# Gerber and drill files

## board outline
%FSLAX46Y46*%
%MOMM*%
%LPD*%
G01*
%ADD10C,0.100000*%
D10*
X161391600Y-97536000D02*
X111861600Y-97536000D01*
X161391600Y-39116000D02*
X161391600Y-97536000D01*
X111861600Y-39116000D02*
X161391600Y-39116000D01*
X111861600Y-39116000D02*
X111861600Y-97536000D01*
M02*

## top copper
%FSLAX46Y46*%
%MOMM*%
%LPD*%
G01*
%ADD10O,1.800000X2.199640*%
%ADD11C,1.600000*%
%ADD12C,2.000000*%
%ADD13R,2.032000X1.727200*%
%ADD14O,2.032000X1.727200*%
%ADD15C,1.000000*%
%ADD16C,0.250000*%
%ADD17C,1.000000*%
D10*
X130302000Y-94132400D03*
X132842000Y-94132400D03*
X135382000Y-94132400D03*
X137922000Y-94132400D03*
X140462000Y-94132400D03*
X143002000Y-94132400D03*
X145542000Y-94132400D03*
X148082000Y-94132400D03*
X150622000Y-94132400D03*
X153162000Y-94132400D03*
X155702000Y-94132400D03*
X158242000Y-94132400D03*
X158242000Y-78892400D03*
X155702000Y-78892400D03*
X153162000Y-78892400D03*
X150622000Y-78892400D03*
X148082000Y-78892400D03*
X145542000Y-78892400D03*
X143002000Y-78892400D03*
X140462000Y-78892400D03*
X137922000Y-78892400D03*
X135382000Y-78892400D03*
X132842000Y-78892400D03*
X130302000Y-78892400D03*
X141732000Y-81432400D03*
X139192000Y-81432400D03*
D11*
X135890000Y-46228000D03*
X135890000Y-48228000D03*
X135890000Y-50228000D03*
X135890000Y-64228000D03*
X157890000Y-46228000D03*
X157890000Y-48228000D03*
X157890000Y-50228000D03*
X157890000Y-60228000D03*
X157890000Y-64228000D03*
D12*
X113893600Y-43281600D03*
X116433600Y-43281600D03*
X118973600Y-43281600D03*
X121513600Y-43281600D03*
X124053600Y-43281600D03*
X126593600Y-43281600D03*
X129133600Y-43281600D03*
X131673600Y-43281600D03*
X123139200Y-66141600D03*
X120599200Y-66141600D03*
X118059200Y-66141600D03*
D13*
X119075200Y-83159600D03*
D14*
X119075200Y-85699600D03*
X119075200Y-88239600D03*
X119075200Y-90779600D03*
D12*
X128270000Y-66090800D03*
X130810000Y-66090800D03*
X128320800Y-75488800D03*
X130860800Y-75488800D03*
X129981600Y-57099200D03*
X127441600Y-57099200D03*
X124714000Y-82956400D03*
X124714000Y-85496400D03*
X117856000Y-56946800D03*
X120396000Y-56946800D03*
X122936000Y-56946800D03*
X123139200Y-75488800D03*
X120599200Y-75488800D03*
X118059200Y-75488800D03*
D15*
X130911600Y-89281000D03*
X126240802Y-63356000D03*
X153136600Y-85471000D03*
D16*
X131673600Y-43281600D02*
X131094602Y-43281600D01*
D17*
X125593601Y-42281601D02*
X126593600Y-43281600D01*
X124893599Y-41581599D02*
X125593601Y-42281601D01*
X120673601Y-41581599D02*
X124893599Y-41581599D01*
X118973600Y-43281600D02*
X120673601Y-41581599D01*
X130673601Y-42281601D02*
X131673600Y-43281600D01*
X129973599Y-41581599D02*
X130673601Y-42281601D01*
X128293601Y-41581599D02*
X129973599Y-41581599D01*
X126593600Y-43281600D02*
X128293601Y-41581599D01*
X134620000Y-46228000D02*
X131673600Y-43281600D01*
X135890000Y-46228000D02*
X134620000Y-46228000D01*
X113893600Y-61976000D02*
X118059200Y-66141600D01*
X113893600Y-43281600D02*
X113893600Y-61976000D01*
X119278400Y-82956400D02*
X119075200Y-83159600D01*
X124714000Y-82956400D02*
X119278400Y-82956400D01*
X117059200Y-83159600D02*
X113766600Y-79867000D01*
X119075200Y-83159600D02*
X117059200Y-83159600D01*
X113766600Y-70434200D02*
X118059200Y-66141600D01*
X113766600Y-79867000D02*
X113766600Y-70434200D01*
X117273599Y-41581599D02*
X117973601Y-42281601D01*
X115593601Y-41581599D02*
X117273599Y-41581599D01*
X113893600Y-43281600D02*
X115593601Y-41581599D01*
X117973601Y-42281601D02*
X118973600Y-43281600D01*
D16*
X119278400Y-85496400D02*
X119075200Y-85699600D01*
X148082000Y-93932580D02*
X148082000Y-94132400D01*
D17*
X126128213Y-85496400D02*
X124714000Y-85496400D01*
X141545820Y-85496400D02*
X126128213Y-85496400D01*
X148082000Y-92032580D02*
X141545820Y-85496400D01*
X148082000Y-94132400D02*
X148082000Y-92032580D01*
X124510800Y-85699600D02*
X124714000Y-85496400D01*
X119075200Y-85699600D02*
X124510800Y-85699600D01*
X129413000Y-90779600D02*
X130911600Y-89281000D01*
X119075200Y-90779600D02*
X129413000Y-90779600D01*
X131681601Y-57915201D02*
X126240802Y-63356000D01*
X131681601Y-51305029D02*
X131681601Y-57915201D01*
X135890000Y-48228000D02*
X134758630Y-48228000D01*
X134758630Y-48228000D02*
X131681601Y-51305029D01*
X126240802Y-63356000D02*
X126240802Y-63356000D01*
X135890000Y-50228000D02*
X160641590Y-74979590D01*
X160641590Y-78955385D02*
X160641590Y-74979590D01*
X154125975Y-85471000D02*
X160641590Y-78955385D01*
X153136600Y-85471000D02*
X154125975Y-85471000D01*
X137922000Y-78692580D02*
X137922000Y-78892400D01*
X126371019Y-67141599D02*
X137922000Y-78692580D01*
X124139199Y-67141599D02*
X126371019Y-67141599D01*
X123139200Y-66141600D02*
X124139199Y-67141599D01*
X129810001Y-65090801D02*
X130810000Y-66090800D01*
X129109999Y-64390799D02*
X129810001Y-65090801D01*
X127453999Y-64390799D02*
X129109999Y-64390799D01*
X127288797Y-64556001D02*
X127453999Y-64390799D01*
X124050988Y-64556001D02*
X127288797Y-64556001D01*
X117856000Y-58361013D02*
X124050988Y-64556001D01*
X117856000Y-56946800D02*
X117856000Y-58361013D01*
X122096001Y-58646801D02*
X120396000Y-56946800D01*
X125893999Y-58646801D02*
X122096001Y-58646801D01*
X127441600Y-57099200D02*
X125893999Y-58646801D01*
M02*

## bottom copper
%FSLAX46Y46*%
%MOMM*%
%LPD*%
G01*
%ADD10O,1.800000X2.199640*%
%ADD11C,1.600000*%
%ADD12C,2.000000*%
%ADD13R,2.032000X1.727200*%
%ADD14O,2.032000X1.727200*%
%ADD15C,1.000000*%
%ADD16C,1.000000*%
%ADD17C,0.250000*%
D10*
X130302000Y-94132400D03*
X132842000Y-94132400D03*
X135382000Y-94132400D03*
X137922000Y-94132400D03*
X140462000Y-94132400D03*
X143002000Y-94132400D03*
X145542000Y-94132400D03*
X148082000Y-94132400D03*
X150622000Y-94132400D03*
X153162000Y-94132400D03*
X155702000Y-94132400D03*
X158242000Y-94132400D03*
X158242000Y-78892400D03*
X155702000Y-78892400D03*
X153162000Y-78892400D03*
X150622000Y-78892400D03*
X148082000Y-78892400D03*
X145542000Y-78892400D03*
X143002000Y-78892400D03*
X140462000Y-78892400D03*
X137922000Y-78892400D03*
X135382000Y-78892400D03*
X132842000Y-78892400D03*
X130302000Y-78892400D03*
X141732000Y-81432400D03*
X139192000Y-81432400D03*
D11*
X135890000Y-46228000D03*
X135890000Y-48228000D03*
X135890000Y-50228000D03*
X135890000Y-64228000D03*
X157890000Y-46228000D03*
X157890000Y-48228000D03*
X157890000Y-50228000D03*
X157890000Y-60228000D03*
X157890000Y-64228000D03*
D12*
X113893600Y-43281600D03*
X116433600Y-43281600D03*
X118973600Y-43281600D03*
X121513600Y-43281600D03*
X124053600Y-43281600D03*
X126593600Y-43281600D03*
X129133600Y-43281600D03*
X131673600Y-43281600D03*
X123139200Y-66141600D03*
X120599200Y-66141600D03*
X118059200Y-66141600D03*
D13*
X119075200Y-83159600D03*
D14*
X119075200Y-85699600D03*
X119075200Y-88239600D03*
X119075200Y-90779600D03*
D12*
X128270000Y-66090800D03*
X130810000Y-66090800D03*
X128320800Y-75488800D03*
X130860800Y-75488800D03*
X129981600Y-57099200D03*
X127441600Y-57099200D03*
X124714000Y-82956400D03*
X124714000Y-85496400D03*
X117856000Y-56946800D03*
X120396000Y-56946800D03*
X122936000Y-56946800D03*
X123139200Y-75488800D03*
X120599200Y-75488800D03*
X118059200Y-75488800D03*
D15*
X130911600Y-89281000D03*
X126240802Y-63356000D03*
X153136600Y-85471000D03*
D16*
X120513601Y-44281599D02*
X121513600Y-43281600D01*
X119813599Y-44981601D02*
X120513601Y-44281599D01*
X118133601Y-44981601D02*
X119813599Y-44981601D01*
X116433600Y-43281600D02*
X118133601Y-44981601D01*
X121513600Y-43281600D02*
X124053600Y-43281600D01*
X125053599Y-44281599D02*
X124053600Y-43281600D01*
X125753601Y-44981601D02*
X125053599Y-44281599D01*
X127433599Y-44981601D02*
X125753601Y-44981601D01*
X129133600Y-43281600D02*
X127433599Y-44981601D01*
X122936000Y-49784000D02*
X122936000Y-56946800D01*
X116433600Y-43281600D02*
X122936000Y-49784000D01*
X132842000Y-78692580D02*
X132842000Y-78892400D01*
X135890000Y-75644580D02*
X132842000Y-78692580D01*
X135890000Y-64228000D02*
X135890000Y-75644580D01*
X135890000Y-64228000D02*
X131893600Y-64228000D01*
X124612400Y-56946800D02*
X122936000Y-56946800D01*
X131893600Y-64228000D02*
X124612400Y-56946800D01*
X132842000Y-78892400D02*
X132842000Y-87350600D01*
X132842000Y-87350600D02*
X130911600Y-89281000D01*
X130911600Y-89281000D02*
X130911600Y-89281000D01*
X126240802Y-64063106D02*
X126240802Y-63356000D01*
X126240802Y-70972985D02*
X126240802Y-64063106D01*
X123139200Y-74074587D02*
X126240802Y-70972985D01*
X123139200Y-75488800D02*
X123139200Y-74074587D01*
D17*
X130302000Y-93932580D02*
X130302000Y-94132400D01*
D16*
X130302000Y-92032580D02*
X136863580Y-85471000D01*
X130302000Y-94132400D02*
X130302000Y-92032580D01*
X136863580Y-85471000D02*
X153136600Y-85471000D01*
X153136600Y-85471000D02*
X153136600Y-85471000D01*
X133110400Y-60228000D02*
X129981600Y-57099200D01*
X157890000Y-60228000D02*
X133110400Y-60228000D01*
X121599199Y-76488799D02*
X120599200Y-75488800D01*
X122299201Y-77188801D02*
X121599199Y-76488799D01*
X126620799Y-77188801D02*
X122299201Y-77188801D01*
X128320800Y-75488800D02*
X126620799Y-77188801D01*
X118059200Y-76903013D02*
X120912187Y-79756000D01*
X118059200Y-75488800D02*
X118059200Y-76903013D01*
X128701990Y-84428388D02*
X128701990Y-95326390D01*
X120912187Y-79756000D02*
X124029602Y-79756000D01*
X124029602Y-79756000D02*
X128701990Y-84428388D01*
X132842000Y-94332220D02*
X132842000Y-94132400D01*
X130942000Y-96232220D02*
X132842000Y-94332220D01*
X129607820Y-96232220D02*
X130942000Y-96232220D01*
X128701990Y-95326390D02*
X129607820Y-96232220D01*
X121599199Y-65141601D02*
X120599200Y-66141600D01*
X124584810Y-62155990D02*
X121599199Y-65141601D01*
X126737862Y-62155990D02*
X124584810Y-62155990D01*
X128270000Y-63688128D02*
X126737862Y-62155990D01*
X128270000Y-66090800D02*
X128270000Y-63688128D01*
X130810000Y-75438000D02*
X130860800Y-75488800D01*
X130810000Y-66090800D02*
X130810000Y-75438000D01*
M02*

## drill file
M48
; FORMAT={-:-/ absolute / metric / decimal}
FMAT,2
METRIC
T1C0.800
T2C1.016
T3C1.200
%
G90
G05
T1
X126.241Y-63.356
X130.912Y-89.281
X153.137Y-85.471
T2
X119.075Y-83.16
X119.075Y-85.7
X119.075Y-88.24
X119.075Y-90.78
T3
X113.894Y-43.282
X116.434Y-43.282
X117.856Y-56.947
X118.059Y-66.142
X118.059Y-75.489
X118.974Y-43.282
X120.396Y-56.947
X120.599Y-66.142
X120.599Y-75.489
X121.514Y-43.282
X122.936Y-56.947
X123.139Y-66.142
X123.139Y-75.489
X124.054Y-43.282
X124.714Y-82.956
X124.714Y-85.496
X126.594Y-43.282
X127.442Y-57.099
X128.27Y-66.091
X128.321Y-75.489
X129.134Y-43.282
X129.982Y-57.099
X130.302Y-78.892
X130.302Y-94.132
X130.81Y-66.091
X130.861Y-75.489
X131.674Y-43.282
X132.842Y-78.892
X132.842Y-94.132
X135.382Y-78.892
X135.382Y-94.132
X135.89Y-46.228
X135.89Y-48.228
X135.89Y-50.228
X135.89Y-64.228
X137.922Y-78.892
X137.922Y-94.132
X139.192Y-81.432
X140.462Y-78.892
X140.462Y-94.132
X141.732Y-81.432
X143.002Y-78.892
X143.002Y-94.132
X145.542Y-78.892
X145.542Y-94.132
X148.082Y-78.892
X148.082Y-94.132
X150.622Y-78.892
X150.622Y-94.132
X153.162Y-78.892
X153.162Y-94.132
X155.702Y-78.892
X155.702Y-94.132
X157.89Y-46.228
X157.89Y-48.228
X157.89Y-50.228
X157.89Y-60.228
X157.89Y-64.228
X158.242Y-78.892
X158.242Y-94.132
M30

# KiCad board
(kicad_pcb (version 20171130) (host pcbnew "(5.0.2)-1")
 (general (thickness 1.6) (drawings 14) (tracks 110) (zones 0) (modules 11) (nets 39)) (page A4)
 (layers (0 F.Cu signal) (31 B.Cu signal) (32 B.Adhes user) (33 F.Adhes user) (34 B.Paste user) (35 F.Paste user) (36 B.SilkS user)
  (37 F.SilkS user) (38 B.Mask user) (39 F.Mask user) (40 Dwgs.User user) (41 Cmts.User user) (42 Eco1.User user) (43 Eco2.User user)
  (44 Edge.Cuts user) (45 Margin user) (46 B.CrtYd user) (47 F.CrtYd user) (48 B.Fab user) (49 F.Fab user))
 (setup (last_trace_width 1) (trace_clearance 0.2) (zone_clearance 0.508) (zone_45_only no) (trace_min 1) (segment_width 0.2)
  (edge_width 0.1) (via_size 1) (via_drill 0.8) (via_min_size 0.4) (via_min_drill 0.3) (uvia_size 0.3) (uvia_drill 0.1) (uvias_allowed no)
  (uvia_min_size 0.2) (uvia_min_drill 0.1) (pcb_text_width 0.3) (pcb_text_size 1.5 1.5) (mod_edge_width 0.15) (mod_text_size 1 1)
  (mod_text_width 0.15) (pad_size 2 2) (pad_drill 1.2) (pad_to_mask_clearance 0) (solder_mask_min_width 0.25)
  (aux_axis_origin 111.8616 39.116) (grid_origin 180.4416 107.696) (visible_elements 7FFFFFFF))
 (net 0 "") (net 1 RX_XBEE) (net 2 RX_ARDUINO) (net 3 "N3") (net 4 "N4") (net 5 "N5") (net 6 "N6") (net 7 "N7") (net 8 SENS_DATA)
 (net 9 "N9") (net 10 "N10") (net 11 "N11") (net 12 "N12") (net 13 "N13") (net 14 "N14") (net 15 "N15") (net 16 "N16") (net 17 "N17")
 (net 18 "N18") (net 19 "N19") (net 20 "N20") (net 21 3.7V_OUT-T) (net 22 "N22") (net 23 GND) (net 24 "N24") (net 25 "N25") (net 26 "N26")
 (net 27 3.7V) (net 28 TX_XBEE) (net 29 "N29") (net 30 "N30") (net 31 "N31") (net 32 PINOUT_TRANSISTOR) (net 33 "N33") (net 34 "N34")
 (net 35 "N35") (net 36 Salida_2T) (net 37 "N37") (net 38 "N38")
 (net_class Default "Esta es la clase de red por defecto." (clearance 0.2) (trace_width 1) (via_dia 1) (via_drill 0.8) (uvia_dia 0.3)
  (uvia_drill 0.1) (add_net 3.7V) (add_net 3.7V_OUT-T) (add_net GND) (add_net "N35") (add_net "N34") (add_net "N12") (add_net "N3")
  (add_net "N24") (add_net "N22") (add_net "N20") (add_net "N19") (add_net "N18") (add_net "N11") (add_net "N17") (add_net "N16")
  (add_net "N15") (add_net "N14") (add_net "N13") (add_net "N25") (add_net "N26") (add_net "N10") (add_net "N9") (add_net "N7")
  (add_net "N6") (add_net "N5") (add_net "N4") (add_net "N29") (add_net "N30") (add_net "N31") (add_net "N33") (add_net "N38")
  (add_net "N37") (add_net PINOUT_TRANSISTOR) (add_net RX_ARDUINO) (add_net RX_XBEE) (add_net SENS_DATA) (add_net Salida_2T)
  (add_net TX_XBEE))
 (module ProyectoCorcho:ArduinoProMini (layer F.Cu) (at 144.272 86.5124)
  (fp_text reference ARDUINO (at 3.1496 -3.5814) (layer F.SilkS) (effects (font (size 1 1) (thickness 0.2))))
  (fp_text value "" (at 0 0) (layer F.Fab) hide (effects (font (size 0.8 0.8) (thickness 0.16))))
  (pad 12 thru_hole oval (at -13.97 7.62) (size 1.8 2.19964) (drill 1.2) (layers *.Cu *.Mask) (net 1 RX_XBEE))
  (pad 11 thru_hole oval (at -11.43 7.62) (size 1.8 2.19964) (drill 1.2) (layers *.Cu *.Mask) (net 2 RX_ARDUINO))
  (pad 10 thru_hole oval (at -8.89 7.62) (size 1.8 2.19964) (drill 1.2) (layers *.Cu *.Mask) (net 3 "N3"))
  (pad 9 thru_hole oval (at -6.35 7.62) (size 1.8 2.19964) (drill 1.2) (layers *.Cu *.Mask) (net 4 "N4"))
  (pad 8 thru_hole oval (at -3.81 7.62) (size 1.8 2.19964) (drill 1.2) (layers *.Cu *.Mask) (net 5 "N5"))
  (pad 7 thru_hole oval (at -1.27 7.62) (size 1.8 2.19964) (drill 1.2) (layers *.Cu *.Mask) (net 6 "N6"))
  (pad 6 thru_hole oval (at 1.27 7.62) (size 1.8 2.19964) (drill 1.2) (layers *.Cu *.Mask) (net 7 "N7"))
  (pad 5 thru_hole oval (at 3.81 7.62) (size 1.8 2.19964) (drill 1.2) (layers *.Cu *.Mask) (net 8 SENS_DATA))
  (pad 4 thru_hole oval (at 6.35 7.62) (size 1.8 2.19964) (drill 1.2) (layers *.Cu *.Mask) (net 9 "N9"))
  (pad 3 thru_hole oval (at 8.89 7.62) (size 1.8 2.19964) (drill 1.2) (layers *.Cu *.Mask) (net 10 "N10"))
  (pad 2 thru_hole oval (at 11.43 7.62) (size 1.8 2.19964) (drill 1.2) (layers *.Cu *.Mask) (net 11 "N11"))
  (pad 1 thru_hole oval (at 13.97 7.62) (size 1.8 2.19964) (drill 1.2) (layers *.Cu *.Mask) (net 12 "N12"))
  (pad 24 thru_hole oval (at 13.97 -7.62) (size 1.8 2.19964) (drill 1.2) (layers *.Cu *.Mask) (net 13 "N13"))
  (pad 23 thru_hole oval (at 11.43 -7.62) (size 1.8 2.19964) (drill 1.2) (layers *.Cu *.Mask) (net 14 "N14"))
  (pad 22 thru_hole oval (at 8.89 -7.62) (size 1.8 2.19964) (drill 1.2) (layers *.Cu *.Mask) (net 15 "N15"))
  (pad 21 thru_hole oval (at 6.35 -7.62) (size 1.8 2.19964) (drill 1.2) (layers *.Cu *.Mask) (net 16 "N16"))
  (pad 20 thru_hole oval (at 3.81 -7.62) (size 1.8 2.19964) (drill 1.2) (layers *.Cu *.Mask) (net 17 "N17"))
  (pad 19 thru_hole oval (at 1.27 -7.62) (size 1.8 2.19964) (drill 1.2) (layers *.Cu *.Mask) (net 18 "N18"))
  (pad 18 thru_hole oval (at -1.27 -7.62) (size 1.8 2.19964) (drill 1.2) (layers *.Cu *.Mask) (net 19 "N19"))
  (pad 17 thru_hole oval (at -3.81 -7.62) (size 1.8 2.19964) (drill 1.2) (layers *.Cu *.Mask) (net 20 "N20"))
  (pad 16 thru_hole oval (at -6.35 -7.62) (size 1.8 2.19964) (drill 1.2) (layers *.Cu *.Mask) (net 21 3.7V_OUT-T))
  (pad 15 thru_hole oval (at -8.89 -7.62) (size 1.8 2.19964) (drill 1.2) (layers *.Cu *.Mask) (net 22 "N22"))
  (pad 14 thru_hole oval (at -11.43 -7.62) (size 1.8 2.19964) (drill 1.2) (layers *.Cu *.Mask) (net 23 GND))
  (pad 13 thru_hole oval (at -13.97 -7.62) (size 1.8 2.19964) (drill 1.2) (layers *.Cu *.Mask) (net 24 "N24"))
  (pad 25 thru_hole oval (at -2.54 -5.08) (size 1.8 2.19964) (drill 1.2) (layers *.Cu *.Mask) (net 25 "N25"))
  (pad 26 thru_hole oval (at -5.08 -5.08) (size 1.8 2.19964) (drill 1.2) (layers *.Cu *.Mask) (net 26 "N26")))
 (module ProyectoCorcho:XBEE (layer F.Cu) (at 134.62 44.958)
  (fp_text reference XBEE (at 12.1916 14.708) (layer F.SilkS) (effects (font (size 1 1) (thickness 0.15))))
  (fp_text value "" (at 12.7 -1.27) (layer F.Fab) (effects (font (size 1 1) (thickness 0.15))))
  (pad 1 thru_hole circle (at 1.27 1.27) (size 1.6 1.6) (drill 1.2) (layers *.Cu *.Mask) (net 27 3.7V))
  (pad 2 thru_hole circle (at 1.27 3.27) (size 1.6 1.6) (drill 1.2) (layers *.Cu *.Mask) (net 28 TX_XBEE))
  (pad 3 thru_hole circle (at 1.27 5.27) (size 1.6 1.6) (drill 1.2) (layers *.Cu *.Mask) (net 1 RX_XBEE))
  (pad 4 thru_hole circle (at 1.27 19.27) (size 1.6 1.6) (drill 1.2) (layers *.Cu *.Mask) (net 23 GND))
  (pad 5 thru_hole circle (at 23.27 1.27) (size 1.6 1.6) (drill 1.2) (layers *.Cu *.Mask) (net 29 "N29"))
  (pad 6 thru_hole circle (at 23.27 3.27) (size 1.6 1.6) (drill 1.2) (layers *.Cu *.Mask) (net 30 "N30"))
  (pad 7 thru_hole circle (at 23.27 5.27) (size 1.6 1.6) (drill 1.2) (layers *.Cu *.Mask) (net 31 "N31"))
  (pad 8 thru_hole circle (at 23.27 15.27) (size 1.6 1.6) (drill 1.2) (layers *.Cu *.Mask) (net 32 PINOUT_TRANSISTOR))
  (pad 9 thru_hole circle (at 23.27 19.27) (size 1.6 1.6) (drill 1.2) (layers *.Cu *.Mask) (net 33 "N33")))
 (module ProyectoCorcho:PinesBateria (layer F.Cu) (at 112.6236 42.0116)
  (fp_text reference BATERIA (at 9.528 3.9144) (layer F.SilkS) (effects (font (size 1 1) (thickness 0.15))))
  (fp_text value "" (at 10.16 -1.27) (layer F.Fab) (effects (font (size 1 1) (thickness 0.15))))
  (pad 1 thru_hole circle (at 1.27 1.27) (size 2 2) (drill 1.2) (layers *.Cu *.Mask) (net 27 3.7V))
  (pad 2 thru_hole circle (at 3.81 1.27) (size 2 2) (drill 1.2) (layers *.Cu *.Mask) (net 23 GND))
  (pad 3 thru_hole circle (at 6.35 1.27) (size 2 2) (drill 1.2) (layers *.Cu *.Mask) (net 27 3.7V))
  (pad 4 thru_hole circle (at 8.89 1.27) (size 2 2) (drill 1.2) (layers *.Cu *.Mask) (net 23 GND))
  (pad 5 thru_hole circle (at 11.43 1.27) (size 2 2) (drill 1.2) (layers *.Cu *.Mask) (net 23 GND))
  (pad 6 thru_hole circle (at 13.97 1.27) (size 2 2) (drill 1.2) (layers *.Cu *.Mask) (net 27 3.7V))
  (pad 7 thru_hole circle (at 16.51 1.27) (size 2 2) (drill 1.2) (layers *.Cu *.Mask) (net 23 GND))
  (pad 8 thru_hole circle (at 19.05 1.27) (size 2 2) (drill 1.2) (layers *.Cu *.Mask) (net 27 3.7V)))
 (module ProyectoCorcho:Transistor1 (layer B.Cu) (at 120.5992 66.1416)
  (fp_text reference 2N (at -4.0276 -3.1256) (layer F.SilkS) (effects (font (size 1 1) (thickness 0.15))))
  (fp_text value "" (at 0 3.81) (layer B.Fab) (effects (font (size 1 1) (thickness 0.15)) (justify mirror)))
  (pad 3 thru_hole circle (at 2.54 0) (size 2 2) (drill 1.2) (layers *.Cu *.Mask) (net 21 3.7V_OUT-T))
  (pad 2 thru_hole circle (at 0 0) (size 2 2) (drill 1.2) (layers *.Cu *.Mask) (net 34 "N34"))
  (pad 1 thru_hole circle (at -2.54 0) (size 2 2) (drill 1.2) (layers *.Cu *.Mask) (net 27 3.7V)))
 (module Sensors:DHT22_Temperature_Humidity (layer F.Cu) (at 119.0752 86.9696 270)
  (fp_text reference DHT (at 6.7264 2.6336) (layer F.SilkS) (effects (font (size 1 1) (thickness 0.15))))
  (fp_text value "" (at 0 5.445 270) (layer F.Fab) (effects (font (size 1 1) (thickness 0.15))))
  (pad 1 thru_hole rect (at -3.81 0) (size 2.032 1.7272) (drill 1.016) (layers *.Cu *.Mask F.SilkS) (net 27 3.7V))
  (pad 2 thru_hole oval (at -1.27 0) (size 2.032 1.7272) (drill 1.016) (layers *.Cu *.Mask F.SilkS) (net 8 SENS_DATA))
  (pad 3 thru_hole oval (at 1.27 0) (size 2.032 1.7272) (drill 1.016) (layers *.Cu *.Mask F.SilkS) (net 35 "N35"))
  (pad 4 thru_hole oval (at 3.81 0) (size 2.032 1.7272) (drill 1.016) (layers *.Cu *.Mask F.SilkS) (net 23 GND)))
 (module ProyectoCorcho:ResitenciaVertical (layer F.Cu) (at 128.27 66.0908)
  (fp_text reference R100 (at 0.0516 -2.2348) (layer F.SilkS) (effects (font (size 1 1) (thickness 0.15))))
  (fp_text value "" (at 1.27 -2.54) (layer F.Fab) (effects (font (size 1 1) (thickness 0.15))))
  (pad 1 thru_hole circle (at 0 0) (size 2 2) (drill 1.2) (layers *.Cu *.Mask) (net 34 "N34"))
  (pad 2 thru_hole circle (at 2.54 0) (size 2 2) (drill 1.2) (layers *.Cu *.Mask) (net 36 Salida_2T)))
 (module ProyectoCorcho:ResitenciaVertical (layer F.Cu) (at 128.3208 75.4888)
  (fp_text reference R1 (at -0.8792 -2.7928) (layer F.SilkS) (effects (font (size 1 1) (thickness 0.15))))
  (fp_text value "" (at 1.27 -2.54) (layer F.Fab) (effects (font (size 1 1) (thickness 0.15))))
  (pad 1 thru_hole circle (at 0 0) (size 2 2) (drill 1.2) (layers *.Cu *.Mask) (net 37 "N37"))
  (pad 2 thru_hole circle (at 2.54 0) (size 2 2) (drill 1.2) (layers *.Cu *.Mask) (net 36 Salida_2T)))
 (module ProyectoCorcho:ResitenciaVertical (layer F.Cu) (at 127.4416 57.0992)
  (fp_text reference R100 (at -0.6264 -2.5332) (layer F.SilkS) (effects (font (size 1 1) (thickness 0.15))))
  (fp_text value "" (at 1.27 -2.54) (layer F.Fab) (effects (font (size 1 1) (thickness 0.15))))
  (pad 2 thru_hole circle (at 2.54 0) (size 2 2) (drill 1.2) (layers *.Cu *.Mask) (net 32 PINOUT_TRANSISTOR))
  (pad 1 thru_hole circle (at 0 0) (size 2 2) (drill 1.2) (layers *.Cu *.Mask) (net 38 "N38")))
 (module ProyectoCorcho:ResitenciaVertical (layer F.Cu) (at 124.714 82.9564 270)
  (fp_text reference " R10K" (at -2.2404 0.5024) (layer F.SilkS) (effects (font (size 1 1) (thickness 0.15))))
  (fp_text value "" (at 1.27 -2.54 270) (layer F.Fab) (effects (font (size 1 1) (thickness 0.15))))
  (pad 1 thru_hole circle (at 0 0 270) (size 2 2) (drill 1.2) (layers *.Cu *.Mask) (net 27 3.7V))
  (pad 2 thru_hole circle (at 2.54 0 270) (size 2 2) (drill 1.2) (layers *.Cu *.Mask) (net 8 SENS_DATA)))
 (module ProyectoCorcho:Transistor (layer F.Cu) (at 120.396 56.9468)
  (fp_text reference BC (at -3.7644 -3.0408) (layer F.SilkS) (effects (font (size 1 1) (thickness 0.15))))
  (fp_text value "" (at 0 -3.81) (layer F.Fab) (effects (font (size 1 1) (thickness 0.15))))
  (pad 1 thru_hole circle (at -2.54 0) (size 2 2) (drill 1.2) (layers *.Cu *.Mask) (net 36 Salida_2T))
  (pad 2 thru_hole circle (at 0 0) (size 2 2) (drill 1.2) (layers *.Cu *.Mask) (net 38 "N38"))
  (pad 3 thru_hole circle (at 2.54 0) (size 2 2) (drill 1.2) (layers *.Cu *.Mask) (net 23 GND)))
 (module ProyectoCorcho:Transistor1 (layer B.Cu) (at 120.5992 75.4888 180)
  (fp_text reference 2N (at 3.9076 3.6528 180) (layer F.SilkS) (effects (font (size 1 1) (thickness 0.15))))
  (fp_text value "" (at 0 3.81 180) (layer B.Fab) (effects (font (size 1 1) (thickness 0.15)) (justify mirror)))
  (pad 1 thru_hole circle (at -2.54 0 180) (size 2 2) (drill 1.2) (layers *.Cu *.Mask) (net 28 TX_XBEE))
  (pad 2 thru_hole circle (at 0 0 180) (size 2 2) (drill 1.2) (layers *.Cu *.Mask) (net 37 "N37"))
  (pad 3 thru_hole circle (at 2.54 0 180) (size 2 2) (drill 1.2) (layers *.Cu *.Mask) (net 2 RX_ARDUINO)))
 (gr_line (start 161.3916 97.536) (end 111.8616 97.536) (layer Edge.Cuts) (width 0.1))
 (gr_line (start 161.3916 39.116) (end 161.3916 97.536) (layer Edge.Cuts) (width 0.1))
 (gr_line (start 111.8616 39.116) (end 161.3916 39.116) (layer Edge.Cuts) (width 0.1))
 (gr_line (start 111.8616 39.116) (end 111.8616 97.536) (layer Edge.Cuts) (width 0.1))
 (segment (start 131.6736 43.2816) (end 131.094602 43.2816) (width 0.25) (layer F.Cu) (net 27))
 (segment (start 125.593601 42.281601) (end 126.5936 43.2816) (width 1) (layer F.Cu) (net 27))
 (segment (start 124.893599 41.581599) (end 125.593601 42.281601) (width 1) (layer F.Cu) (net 27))
 (segment (start 120.673601 41.581599) (end 124.893599 41.581599) (width 1) (layer F.Cu) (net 27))
 (segment (start 118.9736 43.2816) (end 120.673601 41.581599) (width 1) (layer F.Cu) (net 27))
 (segment (start 130.673601 42.281601) (end 131.6736 43.2816) (width 1) (layer F.Cu) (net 27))
 (segment (start 129.973599 41.581599) (end 130.673601 42.281601) (width 1) (layer F.Cu) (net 27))
 (segment (start 128.293601 41.581599) (end 129.973599 41.581599) (width 1) (layer F.Cu) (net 27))
 (segment (start 126.5936 43.2816) (end 128.293601 41.581599) (width 1) (layer F.Cu) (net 27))
 (segment (start 134.62 46.228) (end 131.6736 43.2816) (width 1) (layer F.Cu) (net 27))
 (segment (start 135.89 46.228) (end 134.62 46.228) (width 1) (layer F.Cu) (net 27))
 (segment (start 113.8936 61.976) (end 118.0592 66.1416) (width 1) (layer F.Cu) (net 27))
 (segment (start 113.8936 43.2816) (end 113.8936 61.976) (width 1) (layer F.Cu) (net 27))
 (segment (start 119.2784 82.9564) (end 119.0752 83.1596) (width 1) (layer F.Cu) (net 27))
 (segment (start 124.714 82.9564) (end 119.2784 82.9564) (width 1) (layer F.Cu) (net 27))
 (segment (start 117.0592 83.1596) (end 113.7666 79.867) (width 1) (layer F.Cu) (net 27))
 (segment (start 119.0752 83.1596) (end 117.0592 83.1596) (width 1) (layer F.Cu) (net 27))
 (segment (start 113.7666 70.4342) (end 118.0592 66.1416) (width 1) (layer F.Cu) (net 27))
 (segment (start 113.7666 79.867) (end 113.7666 70.4342) (width 1) (layer F.Cu) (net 27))
 (segment (start 117.273599 41.581599) (end 117.973601 42.281601) (width 1) (layer F.Cu) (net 27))
 (segment (start 115.593601 41.581599) (end 117.273599 41.581599) (width 1) (layer F.Cu) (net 27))
 (segment (start 113.8936 43.2816) (end 115.593601 41.581599) (width 1) (layer F.Cu) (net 27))
 (segment (start 117.973601 42.281601) (end 118.9736 43.2816) (width 1) (layer F.Cu) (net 27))
 (segment (start 119.2784 85.4964) (end 119.0752 85.6996) (width 0.25) (layer F.Cu) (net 8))
 (segment (start 148.082 93.93258) (end 148.082 94.1324) (width 0.25) (layer F.Cu) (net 8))
 (segment (start 126.128213 85.4964) (end 124.714 85.4964) (width 1) (layer F.Cu) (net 8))
 (segment (start 141.54582 85.4964) (end 126.128213 85.4964) (width 1) (layer F.Cu) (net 8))
 (segment (start 148.082 92.03258) (end 141.54582 85.4964) (width 1) (layer F.Cu) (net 8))
 (segment (start 148.082 94.1324) (end 148.082 92.03258) (width 1) (layer F.Cu) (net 8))
 (segment (start 124.5108 85.6996) (end 124.714 85.4964) (width 1) (layer F.Cu) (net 8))
 (segment (start 119.0752 85.6996) (end 124.5108 85.6996) (width 1) (layer F.Cu) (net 8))
 (segment (start 120.513601 44.281599) (end 121.5136 43.2816) (width 1) (layer B.Cu) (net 23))
 (segment (start 119.813599 44.981601) (end 120.513601 44.281599) (width 1) (layer B.Cu) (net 23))
 (segment (start 118.133601 44.981601) (end 119.813599 44.981601) (width 1) (layer B.Cu) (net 23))
 (segment (start 116.4336 43.2816) (end 118.133601 44.981601) (width 1) (layer B.Cu) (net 23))
 (segment (start 121.5136 43.2816) (end 124.0536 43.2816) (width 1) (layer B.Cu) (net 23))
 (segment (start 125.053599 44.281599) (end 124.0536 43.2816) (width 1) (layer B.Cu) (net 23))
 (segment (start 125.753601 44.981601) (end 125.053599 44.281599) (width 1) (layer B.Cu) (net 23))
 (segment (start 127.433599 44.981601) (end 125.753601 44.981601) (width 1) (layer B.Cu) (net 23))
 (segment (start 129.1336 43.2816) (end 127.433599 44.981601) (width 1) (layer B.Cu) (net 23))
 (segment (start 122.936 49.784) (end 122.936 56.9468) (width 1) (layer B.Cu) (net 23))
 (segment (start 116.4336 43.2816) (end 122.936 49.784) (width 1) (layer B.Cu) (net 23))
 (segment (start 132.842 78.69258) (end 132.842 78.8924) (width 1) (layer B.Cu) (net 23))
 (segment (start 135.89 75.64458) (end 132.842 78.69258) (width 1) (layer B.Cu) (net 23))
 (segment (start 135.89 64.228) (end 135.89 75.64458) (width 1) (layer B.Cu) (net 23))
 (segment (start 135.89 64.228) (end 131.8936 64.228) (width 1) (layer B.Cu) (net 23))
 (segment (start 124.6124 56.9468) (end 122.936 56.9468) (width 1) (layer B.Cu) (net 23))
 (segment (start 131.8936 64.228) (end 124.6124 56.9468) (width 1) (layer B.Cu) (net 23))
 (segment (start 132.842 78.8924) (end 132.842 87.3506) (width 1) (layer B.Cu) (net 23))
 (segment (start 132.842 87.3506) (end 130.9116 89.281) (width 1) (layer B.Cu) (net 23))
 (segment (start 130.9116 89.281) (end 130.9116 89.281) (width 1) (layer B.Cu) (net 23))
 (via (at 130.9116 89.281) (size 1) (drill 0.8) (layers F.Cu B.Cu) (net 23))
 (segment (start 129.413 90.7796) (end 130.9116 89.281) (width 1) (layer F.Cu) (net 23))
 (segment (start 119.0752 90.7796) (end 129.413 90.7796) (width 1) (layer F.Cu) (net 23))
 (segment (start 131.681601 57.915201) (end 126.240802 63.356) (width 1) (layer F.Cu) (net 28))
 (segment (start 131.681601 51.305029) (end 131.681601 57.915201) (width 1) (layer F.Cu) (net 28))
 (segment (start 135.89 48.228) (end 134.75863 48.228) (width 1) (layer F.Cu) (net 28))
 (segment (start 134.75863 48.228) (end 131.681601 51.305029) (width 1) (layer F.Cu) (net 28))
 (segment (start 126.240802 63.356) (end 126.240802 63.356) (width 1) (layer F.Cu) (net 28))
 (via (at 126.240802 63.356) (size 1) (drill 0.8) (layers F.Cu B.Cu) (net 28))
 (segment (start 126.240802 64.063106) (end 126.240802 63.356) (width 1) (layer B.Cu) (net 28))
 (segment (start 126.240802 70.972985) (end 126.240802 64.063106) (width 1) (layer B.Cu) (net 28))
 (segment (start 123.1392 74.074587) (end 126.240802 70.972985) (width 1) (layer B.Cu) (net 28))
 (segment (start 123.1392 75.4888) (end 123.1392 74.074587) (width 1) (layer B.Cu) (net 28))
 (segment (start 130.302 93.93258) (end 130.302 94.1324) (width 0.25) (layer B.Cu) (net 1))
 (segment (start 135.89 50.228) (end 160.64159 74.97959) (width 1) (layer F.Cu) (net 1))
 (segment (start 130.302 92.03258) (end 136.86358 85.471) (width 1) (layer B.Cu) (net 1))
 (segment (start 130.302 94.1324) (end 130.302 92.03258) (width 1) (layer B.Cu) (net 1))
 (segment (start 136.86358 85.471) (end 153.1366 85.471) (width 1) (layer B.Cu) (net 1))
 (segment (start 153.1366 85.471) (end 153.1366 85.471) (width 1) (layer B.Cu) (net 1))
 (via (at 153.1366 85.471) (size 1) (drill 0.8) (layers F.Cu B.Cu) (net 1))
 (segment (start 160.64159 78.955385) (end 160.64159 74.97959) (width 1) (layer F.Cu) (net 1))
 (segment (start 154.125975 85.471) (end 160.64159 78.955385) (width 1) (layer F.Cu) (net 1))
 (segment (start 153.1366 85.471) (end 154.125975 85.471) (width 1) (layer F.Cu) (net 1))
 (segment (start 133.1104 60.228) (end 129.9816 57.0992) (width 1) (layer B.Cu) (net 32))
 (segment (start 157.89 60.228) (end 133.1104 60.228) (width 1) (layer B.Cu) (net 32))
 (segment (start 121.599199 76.488799) (end 120.5992 75.4888) (width 1) (layer B.Cu) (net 37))
 (segment (start 122.299201 77.188801) (end 121.599199 76.488799) (width 1) (layer B.Cu) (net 37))
 (segment (start 126.620799 77.188801) (end 122.299201 77.188801) (width 1) (layer B.Cu) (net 37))
 (segment (start 128.3208 75.4888) (end 126.620799 77.188801) (width 1) (layer B.Cu) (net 37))
 (segment (start 118.0592 76.903013) (end 120.912187 79.756) (width 1) (layer B.Cu) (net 2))
 (segment (start 118.0592 75.4888) (end 118.0592 76.903013) (width 1) (layer B.Cu) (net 2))
 (segment (start 128.70199 84.428388) (end 128.70199 95.32639) (width 1) (layer B.Cu) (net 2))
 (segment (start 120.912187 79.756) (end 124.029602 79.756) (width 1) (layer B.Cu) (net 2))
 (segment (start 124.029602 79.756) (end 128.70199 84.428388) (width 1) (layer B.Cu) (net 2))
 (segment (start 132.842 94.33222) (end 132.842 94.1324) (width 1) (layer B.Cu) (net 2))
 (segment (start 130.942 96.23222) (end 132.842 94.33222) (width 1) (layer B.Cu) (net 2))
 (segment (start 129.60782 96.23222) (end 130.942 96.23222) (width 1) (layer B.Cu) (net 2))
 (segment (start 128.70199 95.32639) (end 129.60782 96.23222) (width 1) (layer B.Cu) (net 2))
 (segment (start 137.922 78.69258) (end 137.922 78.8924) (width 1) (layer F.Cu) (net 21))
 (segment (start 126.371019 67.141599) (end 137.922 78.69258) (width 1) (layer F.Cu) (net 21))
 (segment (start 124.139199 67.141599) (end 126.371019 67.141599) (width 1) (layer F.Cu) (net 21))
 (segment (start 123.1392 66.1416) (end 124.139199 67.141599) (width 1) (layer F.Cu) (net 21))
 (segment (start 121.599199 65.141601) (end 120.5992 66.1416) (width 1) (layer B.Cu) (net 34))
 (segment (start 124.58481 62.15599) (end 121.599199 65.141601) (width 1) (layer B.Cu) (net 34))
 (segment (start 126.737862 62.15599) (end 124.58481 62.15599) (width 1) (layer B.Cu) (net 34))
 (segment (start 128.27 63.688128) (end 126.737862 62.15599) (width 1) (layer B.Cu) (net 34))
 (segment (start 128.27 66.0908) (end 128.27 63.688128) (width 1) (layer B.Cu) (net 34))
 (segment (start 129.810001 65.090801) (end 130.81 66.0908) (width 1) (layer F.Cu) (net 36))
 (segment (start 129.109999 64.390799) (end 129.810001 65.090801) (width 1) (layer F.Cu) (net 36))
 (segment (start 127.453999 64.390799) (end 129.109999 64.390799) (width 1) (layer F.Cu) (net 36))
 (segment (start 127.288797 64.556001) (end 127.453999 64.390799) (width 1) (layer F.Cu) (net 36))
 (segment (start 124.050988 64.556001) (end 127.288797 64.556001) (width 1) (layer F.Cu) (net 36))
 (segment (start 117.856 58.361013) (end 124.050988 64.556001) (width 1) (layer F.Cu) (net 36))
 (segment (start 117.856 56.9468) (end 117.856 58.361013) (width 1) (layer F.Cu) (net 36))
 (segment (start 130.81 75.438) (end 130.8608 75.4888) (width 1) (layer B.Cu) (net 36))
 (segment (start 130.81 66.0908) (end 130.81 75.438) (width 1) (layer B.Cu) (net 36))
 (segment (start 122.096001 58.646801) (end 120.396 56.9468) (width 1) (layer F.Cu) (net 38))
 (segment (start 125.893999 58.646801) (end 122.096001 58.646801) (width 1) (layer F.Cu) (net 38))
 (segment (start 127.4416 57.0992) (end 125.893999 58.646801) (width 1) (layer F.Cu) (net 38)))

